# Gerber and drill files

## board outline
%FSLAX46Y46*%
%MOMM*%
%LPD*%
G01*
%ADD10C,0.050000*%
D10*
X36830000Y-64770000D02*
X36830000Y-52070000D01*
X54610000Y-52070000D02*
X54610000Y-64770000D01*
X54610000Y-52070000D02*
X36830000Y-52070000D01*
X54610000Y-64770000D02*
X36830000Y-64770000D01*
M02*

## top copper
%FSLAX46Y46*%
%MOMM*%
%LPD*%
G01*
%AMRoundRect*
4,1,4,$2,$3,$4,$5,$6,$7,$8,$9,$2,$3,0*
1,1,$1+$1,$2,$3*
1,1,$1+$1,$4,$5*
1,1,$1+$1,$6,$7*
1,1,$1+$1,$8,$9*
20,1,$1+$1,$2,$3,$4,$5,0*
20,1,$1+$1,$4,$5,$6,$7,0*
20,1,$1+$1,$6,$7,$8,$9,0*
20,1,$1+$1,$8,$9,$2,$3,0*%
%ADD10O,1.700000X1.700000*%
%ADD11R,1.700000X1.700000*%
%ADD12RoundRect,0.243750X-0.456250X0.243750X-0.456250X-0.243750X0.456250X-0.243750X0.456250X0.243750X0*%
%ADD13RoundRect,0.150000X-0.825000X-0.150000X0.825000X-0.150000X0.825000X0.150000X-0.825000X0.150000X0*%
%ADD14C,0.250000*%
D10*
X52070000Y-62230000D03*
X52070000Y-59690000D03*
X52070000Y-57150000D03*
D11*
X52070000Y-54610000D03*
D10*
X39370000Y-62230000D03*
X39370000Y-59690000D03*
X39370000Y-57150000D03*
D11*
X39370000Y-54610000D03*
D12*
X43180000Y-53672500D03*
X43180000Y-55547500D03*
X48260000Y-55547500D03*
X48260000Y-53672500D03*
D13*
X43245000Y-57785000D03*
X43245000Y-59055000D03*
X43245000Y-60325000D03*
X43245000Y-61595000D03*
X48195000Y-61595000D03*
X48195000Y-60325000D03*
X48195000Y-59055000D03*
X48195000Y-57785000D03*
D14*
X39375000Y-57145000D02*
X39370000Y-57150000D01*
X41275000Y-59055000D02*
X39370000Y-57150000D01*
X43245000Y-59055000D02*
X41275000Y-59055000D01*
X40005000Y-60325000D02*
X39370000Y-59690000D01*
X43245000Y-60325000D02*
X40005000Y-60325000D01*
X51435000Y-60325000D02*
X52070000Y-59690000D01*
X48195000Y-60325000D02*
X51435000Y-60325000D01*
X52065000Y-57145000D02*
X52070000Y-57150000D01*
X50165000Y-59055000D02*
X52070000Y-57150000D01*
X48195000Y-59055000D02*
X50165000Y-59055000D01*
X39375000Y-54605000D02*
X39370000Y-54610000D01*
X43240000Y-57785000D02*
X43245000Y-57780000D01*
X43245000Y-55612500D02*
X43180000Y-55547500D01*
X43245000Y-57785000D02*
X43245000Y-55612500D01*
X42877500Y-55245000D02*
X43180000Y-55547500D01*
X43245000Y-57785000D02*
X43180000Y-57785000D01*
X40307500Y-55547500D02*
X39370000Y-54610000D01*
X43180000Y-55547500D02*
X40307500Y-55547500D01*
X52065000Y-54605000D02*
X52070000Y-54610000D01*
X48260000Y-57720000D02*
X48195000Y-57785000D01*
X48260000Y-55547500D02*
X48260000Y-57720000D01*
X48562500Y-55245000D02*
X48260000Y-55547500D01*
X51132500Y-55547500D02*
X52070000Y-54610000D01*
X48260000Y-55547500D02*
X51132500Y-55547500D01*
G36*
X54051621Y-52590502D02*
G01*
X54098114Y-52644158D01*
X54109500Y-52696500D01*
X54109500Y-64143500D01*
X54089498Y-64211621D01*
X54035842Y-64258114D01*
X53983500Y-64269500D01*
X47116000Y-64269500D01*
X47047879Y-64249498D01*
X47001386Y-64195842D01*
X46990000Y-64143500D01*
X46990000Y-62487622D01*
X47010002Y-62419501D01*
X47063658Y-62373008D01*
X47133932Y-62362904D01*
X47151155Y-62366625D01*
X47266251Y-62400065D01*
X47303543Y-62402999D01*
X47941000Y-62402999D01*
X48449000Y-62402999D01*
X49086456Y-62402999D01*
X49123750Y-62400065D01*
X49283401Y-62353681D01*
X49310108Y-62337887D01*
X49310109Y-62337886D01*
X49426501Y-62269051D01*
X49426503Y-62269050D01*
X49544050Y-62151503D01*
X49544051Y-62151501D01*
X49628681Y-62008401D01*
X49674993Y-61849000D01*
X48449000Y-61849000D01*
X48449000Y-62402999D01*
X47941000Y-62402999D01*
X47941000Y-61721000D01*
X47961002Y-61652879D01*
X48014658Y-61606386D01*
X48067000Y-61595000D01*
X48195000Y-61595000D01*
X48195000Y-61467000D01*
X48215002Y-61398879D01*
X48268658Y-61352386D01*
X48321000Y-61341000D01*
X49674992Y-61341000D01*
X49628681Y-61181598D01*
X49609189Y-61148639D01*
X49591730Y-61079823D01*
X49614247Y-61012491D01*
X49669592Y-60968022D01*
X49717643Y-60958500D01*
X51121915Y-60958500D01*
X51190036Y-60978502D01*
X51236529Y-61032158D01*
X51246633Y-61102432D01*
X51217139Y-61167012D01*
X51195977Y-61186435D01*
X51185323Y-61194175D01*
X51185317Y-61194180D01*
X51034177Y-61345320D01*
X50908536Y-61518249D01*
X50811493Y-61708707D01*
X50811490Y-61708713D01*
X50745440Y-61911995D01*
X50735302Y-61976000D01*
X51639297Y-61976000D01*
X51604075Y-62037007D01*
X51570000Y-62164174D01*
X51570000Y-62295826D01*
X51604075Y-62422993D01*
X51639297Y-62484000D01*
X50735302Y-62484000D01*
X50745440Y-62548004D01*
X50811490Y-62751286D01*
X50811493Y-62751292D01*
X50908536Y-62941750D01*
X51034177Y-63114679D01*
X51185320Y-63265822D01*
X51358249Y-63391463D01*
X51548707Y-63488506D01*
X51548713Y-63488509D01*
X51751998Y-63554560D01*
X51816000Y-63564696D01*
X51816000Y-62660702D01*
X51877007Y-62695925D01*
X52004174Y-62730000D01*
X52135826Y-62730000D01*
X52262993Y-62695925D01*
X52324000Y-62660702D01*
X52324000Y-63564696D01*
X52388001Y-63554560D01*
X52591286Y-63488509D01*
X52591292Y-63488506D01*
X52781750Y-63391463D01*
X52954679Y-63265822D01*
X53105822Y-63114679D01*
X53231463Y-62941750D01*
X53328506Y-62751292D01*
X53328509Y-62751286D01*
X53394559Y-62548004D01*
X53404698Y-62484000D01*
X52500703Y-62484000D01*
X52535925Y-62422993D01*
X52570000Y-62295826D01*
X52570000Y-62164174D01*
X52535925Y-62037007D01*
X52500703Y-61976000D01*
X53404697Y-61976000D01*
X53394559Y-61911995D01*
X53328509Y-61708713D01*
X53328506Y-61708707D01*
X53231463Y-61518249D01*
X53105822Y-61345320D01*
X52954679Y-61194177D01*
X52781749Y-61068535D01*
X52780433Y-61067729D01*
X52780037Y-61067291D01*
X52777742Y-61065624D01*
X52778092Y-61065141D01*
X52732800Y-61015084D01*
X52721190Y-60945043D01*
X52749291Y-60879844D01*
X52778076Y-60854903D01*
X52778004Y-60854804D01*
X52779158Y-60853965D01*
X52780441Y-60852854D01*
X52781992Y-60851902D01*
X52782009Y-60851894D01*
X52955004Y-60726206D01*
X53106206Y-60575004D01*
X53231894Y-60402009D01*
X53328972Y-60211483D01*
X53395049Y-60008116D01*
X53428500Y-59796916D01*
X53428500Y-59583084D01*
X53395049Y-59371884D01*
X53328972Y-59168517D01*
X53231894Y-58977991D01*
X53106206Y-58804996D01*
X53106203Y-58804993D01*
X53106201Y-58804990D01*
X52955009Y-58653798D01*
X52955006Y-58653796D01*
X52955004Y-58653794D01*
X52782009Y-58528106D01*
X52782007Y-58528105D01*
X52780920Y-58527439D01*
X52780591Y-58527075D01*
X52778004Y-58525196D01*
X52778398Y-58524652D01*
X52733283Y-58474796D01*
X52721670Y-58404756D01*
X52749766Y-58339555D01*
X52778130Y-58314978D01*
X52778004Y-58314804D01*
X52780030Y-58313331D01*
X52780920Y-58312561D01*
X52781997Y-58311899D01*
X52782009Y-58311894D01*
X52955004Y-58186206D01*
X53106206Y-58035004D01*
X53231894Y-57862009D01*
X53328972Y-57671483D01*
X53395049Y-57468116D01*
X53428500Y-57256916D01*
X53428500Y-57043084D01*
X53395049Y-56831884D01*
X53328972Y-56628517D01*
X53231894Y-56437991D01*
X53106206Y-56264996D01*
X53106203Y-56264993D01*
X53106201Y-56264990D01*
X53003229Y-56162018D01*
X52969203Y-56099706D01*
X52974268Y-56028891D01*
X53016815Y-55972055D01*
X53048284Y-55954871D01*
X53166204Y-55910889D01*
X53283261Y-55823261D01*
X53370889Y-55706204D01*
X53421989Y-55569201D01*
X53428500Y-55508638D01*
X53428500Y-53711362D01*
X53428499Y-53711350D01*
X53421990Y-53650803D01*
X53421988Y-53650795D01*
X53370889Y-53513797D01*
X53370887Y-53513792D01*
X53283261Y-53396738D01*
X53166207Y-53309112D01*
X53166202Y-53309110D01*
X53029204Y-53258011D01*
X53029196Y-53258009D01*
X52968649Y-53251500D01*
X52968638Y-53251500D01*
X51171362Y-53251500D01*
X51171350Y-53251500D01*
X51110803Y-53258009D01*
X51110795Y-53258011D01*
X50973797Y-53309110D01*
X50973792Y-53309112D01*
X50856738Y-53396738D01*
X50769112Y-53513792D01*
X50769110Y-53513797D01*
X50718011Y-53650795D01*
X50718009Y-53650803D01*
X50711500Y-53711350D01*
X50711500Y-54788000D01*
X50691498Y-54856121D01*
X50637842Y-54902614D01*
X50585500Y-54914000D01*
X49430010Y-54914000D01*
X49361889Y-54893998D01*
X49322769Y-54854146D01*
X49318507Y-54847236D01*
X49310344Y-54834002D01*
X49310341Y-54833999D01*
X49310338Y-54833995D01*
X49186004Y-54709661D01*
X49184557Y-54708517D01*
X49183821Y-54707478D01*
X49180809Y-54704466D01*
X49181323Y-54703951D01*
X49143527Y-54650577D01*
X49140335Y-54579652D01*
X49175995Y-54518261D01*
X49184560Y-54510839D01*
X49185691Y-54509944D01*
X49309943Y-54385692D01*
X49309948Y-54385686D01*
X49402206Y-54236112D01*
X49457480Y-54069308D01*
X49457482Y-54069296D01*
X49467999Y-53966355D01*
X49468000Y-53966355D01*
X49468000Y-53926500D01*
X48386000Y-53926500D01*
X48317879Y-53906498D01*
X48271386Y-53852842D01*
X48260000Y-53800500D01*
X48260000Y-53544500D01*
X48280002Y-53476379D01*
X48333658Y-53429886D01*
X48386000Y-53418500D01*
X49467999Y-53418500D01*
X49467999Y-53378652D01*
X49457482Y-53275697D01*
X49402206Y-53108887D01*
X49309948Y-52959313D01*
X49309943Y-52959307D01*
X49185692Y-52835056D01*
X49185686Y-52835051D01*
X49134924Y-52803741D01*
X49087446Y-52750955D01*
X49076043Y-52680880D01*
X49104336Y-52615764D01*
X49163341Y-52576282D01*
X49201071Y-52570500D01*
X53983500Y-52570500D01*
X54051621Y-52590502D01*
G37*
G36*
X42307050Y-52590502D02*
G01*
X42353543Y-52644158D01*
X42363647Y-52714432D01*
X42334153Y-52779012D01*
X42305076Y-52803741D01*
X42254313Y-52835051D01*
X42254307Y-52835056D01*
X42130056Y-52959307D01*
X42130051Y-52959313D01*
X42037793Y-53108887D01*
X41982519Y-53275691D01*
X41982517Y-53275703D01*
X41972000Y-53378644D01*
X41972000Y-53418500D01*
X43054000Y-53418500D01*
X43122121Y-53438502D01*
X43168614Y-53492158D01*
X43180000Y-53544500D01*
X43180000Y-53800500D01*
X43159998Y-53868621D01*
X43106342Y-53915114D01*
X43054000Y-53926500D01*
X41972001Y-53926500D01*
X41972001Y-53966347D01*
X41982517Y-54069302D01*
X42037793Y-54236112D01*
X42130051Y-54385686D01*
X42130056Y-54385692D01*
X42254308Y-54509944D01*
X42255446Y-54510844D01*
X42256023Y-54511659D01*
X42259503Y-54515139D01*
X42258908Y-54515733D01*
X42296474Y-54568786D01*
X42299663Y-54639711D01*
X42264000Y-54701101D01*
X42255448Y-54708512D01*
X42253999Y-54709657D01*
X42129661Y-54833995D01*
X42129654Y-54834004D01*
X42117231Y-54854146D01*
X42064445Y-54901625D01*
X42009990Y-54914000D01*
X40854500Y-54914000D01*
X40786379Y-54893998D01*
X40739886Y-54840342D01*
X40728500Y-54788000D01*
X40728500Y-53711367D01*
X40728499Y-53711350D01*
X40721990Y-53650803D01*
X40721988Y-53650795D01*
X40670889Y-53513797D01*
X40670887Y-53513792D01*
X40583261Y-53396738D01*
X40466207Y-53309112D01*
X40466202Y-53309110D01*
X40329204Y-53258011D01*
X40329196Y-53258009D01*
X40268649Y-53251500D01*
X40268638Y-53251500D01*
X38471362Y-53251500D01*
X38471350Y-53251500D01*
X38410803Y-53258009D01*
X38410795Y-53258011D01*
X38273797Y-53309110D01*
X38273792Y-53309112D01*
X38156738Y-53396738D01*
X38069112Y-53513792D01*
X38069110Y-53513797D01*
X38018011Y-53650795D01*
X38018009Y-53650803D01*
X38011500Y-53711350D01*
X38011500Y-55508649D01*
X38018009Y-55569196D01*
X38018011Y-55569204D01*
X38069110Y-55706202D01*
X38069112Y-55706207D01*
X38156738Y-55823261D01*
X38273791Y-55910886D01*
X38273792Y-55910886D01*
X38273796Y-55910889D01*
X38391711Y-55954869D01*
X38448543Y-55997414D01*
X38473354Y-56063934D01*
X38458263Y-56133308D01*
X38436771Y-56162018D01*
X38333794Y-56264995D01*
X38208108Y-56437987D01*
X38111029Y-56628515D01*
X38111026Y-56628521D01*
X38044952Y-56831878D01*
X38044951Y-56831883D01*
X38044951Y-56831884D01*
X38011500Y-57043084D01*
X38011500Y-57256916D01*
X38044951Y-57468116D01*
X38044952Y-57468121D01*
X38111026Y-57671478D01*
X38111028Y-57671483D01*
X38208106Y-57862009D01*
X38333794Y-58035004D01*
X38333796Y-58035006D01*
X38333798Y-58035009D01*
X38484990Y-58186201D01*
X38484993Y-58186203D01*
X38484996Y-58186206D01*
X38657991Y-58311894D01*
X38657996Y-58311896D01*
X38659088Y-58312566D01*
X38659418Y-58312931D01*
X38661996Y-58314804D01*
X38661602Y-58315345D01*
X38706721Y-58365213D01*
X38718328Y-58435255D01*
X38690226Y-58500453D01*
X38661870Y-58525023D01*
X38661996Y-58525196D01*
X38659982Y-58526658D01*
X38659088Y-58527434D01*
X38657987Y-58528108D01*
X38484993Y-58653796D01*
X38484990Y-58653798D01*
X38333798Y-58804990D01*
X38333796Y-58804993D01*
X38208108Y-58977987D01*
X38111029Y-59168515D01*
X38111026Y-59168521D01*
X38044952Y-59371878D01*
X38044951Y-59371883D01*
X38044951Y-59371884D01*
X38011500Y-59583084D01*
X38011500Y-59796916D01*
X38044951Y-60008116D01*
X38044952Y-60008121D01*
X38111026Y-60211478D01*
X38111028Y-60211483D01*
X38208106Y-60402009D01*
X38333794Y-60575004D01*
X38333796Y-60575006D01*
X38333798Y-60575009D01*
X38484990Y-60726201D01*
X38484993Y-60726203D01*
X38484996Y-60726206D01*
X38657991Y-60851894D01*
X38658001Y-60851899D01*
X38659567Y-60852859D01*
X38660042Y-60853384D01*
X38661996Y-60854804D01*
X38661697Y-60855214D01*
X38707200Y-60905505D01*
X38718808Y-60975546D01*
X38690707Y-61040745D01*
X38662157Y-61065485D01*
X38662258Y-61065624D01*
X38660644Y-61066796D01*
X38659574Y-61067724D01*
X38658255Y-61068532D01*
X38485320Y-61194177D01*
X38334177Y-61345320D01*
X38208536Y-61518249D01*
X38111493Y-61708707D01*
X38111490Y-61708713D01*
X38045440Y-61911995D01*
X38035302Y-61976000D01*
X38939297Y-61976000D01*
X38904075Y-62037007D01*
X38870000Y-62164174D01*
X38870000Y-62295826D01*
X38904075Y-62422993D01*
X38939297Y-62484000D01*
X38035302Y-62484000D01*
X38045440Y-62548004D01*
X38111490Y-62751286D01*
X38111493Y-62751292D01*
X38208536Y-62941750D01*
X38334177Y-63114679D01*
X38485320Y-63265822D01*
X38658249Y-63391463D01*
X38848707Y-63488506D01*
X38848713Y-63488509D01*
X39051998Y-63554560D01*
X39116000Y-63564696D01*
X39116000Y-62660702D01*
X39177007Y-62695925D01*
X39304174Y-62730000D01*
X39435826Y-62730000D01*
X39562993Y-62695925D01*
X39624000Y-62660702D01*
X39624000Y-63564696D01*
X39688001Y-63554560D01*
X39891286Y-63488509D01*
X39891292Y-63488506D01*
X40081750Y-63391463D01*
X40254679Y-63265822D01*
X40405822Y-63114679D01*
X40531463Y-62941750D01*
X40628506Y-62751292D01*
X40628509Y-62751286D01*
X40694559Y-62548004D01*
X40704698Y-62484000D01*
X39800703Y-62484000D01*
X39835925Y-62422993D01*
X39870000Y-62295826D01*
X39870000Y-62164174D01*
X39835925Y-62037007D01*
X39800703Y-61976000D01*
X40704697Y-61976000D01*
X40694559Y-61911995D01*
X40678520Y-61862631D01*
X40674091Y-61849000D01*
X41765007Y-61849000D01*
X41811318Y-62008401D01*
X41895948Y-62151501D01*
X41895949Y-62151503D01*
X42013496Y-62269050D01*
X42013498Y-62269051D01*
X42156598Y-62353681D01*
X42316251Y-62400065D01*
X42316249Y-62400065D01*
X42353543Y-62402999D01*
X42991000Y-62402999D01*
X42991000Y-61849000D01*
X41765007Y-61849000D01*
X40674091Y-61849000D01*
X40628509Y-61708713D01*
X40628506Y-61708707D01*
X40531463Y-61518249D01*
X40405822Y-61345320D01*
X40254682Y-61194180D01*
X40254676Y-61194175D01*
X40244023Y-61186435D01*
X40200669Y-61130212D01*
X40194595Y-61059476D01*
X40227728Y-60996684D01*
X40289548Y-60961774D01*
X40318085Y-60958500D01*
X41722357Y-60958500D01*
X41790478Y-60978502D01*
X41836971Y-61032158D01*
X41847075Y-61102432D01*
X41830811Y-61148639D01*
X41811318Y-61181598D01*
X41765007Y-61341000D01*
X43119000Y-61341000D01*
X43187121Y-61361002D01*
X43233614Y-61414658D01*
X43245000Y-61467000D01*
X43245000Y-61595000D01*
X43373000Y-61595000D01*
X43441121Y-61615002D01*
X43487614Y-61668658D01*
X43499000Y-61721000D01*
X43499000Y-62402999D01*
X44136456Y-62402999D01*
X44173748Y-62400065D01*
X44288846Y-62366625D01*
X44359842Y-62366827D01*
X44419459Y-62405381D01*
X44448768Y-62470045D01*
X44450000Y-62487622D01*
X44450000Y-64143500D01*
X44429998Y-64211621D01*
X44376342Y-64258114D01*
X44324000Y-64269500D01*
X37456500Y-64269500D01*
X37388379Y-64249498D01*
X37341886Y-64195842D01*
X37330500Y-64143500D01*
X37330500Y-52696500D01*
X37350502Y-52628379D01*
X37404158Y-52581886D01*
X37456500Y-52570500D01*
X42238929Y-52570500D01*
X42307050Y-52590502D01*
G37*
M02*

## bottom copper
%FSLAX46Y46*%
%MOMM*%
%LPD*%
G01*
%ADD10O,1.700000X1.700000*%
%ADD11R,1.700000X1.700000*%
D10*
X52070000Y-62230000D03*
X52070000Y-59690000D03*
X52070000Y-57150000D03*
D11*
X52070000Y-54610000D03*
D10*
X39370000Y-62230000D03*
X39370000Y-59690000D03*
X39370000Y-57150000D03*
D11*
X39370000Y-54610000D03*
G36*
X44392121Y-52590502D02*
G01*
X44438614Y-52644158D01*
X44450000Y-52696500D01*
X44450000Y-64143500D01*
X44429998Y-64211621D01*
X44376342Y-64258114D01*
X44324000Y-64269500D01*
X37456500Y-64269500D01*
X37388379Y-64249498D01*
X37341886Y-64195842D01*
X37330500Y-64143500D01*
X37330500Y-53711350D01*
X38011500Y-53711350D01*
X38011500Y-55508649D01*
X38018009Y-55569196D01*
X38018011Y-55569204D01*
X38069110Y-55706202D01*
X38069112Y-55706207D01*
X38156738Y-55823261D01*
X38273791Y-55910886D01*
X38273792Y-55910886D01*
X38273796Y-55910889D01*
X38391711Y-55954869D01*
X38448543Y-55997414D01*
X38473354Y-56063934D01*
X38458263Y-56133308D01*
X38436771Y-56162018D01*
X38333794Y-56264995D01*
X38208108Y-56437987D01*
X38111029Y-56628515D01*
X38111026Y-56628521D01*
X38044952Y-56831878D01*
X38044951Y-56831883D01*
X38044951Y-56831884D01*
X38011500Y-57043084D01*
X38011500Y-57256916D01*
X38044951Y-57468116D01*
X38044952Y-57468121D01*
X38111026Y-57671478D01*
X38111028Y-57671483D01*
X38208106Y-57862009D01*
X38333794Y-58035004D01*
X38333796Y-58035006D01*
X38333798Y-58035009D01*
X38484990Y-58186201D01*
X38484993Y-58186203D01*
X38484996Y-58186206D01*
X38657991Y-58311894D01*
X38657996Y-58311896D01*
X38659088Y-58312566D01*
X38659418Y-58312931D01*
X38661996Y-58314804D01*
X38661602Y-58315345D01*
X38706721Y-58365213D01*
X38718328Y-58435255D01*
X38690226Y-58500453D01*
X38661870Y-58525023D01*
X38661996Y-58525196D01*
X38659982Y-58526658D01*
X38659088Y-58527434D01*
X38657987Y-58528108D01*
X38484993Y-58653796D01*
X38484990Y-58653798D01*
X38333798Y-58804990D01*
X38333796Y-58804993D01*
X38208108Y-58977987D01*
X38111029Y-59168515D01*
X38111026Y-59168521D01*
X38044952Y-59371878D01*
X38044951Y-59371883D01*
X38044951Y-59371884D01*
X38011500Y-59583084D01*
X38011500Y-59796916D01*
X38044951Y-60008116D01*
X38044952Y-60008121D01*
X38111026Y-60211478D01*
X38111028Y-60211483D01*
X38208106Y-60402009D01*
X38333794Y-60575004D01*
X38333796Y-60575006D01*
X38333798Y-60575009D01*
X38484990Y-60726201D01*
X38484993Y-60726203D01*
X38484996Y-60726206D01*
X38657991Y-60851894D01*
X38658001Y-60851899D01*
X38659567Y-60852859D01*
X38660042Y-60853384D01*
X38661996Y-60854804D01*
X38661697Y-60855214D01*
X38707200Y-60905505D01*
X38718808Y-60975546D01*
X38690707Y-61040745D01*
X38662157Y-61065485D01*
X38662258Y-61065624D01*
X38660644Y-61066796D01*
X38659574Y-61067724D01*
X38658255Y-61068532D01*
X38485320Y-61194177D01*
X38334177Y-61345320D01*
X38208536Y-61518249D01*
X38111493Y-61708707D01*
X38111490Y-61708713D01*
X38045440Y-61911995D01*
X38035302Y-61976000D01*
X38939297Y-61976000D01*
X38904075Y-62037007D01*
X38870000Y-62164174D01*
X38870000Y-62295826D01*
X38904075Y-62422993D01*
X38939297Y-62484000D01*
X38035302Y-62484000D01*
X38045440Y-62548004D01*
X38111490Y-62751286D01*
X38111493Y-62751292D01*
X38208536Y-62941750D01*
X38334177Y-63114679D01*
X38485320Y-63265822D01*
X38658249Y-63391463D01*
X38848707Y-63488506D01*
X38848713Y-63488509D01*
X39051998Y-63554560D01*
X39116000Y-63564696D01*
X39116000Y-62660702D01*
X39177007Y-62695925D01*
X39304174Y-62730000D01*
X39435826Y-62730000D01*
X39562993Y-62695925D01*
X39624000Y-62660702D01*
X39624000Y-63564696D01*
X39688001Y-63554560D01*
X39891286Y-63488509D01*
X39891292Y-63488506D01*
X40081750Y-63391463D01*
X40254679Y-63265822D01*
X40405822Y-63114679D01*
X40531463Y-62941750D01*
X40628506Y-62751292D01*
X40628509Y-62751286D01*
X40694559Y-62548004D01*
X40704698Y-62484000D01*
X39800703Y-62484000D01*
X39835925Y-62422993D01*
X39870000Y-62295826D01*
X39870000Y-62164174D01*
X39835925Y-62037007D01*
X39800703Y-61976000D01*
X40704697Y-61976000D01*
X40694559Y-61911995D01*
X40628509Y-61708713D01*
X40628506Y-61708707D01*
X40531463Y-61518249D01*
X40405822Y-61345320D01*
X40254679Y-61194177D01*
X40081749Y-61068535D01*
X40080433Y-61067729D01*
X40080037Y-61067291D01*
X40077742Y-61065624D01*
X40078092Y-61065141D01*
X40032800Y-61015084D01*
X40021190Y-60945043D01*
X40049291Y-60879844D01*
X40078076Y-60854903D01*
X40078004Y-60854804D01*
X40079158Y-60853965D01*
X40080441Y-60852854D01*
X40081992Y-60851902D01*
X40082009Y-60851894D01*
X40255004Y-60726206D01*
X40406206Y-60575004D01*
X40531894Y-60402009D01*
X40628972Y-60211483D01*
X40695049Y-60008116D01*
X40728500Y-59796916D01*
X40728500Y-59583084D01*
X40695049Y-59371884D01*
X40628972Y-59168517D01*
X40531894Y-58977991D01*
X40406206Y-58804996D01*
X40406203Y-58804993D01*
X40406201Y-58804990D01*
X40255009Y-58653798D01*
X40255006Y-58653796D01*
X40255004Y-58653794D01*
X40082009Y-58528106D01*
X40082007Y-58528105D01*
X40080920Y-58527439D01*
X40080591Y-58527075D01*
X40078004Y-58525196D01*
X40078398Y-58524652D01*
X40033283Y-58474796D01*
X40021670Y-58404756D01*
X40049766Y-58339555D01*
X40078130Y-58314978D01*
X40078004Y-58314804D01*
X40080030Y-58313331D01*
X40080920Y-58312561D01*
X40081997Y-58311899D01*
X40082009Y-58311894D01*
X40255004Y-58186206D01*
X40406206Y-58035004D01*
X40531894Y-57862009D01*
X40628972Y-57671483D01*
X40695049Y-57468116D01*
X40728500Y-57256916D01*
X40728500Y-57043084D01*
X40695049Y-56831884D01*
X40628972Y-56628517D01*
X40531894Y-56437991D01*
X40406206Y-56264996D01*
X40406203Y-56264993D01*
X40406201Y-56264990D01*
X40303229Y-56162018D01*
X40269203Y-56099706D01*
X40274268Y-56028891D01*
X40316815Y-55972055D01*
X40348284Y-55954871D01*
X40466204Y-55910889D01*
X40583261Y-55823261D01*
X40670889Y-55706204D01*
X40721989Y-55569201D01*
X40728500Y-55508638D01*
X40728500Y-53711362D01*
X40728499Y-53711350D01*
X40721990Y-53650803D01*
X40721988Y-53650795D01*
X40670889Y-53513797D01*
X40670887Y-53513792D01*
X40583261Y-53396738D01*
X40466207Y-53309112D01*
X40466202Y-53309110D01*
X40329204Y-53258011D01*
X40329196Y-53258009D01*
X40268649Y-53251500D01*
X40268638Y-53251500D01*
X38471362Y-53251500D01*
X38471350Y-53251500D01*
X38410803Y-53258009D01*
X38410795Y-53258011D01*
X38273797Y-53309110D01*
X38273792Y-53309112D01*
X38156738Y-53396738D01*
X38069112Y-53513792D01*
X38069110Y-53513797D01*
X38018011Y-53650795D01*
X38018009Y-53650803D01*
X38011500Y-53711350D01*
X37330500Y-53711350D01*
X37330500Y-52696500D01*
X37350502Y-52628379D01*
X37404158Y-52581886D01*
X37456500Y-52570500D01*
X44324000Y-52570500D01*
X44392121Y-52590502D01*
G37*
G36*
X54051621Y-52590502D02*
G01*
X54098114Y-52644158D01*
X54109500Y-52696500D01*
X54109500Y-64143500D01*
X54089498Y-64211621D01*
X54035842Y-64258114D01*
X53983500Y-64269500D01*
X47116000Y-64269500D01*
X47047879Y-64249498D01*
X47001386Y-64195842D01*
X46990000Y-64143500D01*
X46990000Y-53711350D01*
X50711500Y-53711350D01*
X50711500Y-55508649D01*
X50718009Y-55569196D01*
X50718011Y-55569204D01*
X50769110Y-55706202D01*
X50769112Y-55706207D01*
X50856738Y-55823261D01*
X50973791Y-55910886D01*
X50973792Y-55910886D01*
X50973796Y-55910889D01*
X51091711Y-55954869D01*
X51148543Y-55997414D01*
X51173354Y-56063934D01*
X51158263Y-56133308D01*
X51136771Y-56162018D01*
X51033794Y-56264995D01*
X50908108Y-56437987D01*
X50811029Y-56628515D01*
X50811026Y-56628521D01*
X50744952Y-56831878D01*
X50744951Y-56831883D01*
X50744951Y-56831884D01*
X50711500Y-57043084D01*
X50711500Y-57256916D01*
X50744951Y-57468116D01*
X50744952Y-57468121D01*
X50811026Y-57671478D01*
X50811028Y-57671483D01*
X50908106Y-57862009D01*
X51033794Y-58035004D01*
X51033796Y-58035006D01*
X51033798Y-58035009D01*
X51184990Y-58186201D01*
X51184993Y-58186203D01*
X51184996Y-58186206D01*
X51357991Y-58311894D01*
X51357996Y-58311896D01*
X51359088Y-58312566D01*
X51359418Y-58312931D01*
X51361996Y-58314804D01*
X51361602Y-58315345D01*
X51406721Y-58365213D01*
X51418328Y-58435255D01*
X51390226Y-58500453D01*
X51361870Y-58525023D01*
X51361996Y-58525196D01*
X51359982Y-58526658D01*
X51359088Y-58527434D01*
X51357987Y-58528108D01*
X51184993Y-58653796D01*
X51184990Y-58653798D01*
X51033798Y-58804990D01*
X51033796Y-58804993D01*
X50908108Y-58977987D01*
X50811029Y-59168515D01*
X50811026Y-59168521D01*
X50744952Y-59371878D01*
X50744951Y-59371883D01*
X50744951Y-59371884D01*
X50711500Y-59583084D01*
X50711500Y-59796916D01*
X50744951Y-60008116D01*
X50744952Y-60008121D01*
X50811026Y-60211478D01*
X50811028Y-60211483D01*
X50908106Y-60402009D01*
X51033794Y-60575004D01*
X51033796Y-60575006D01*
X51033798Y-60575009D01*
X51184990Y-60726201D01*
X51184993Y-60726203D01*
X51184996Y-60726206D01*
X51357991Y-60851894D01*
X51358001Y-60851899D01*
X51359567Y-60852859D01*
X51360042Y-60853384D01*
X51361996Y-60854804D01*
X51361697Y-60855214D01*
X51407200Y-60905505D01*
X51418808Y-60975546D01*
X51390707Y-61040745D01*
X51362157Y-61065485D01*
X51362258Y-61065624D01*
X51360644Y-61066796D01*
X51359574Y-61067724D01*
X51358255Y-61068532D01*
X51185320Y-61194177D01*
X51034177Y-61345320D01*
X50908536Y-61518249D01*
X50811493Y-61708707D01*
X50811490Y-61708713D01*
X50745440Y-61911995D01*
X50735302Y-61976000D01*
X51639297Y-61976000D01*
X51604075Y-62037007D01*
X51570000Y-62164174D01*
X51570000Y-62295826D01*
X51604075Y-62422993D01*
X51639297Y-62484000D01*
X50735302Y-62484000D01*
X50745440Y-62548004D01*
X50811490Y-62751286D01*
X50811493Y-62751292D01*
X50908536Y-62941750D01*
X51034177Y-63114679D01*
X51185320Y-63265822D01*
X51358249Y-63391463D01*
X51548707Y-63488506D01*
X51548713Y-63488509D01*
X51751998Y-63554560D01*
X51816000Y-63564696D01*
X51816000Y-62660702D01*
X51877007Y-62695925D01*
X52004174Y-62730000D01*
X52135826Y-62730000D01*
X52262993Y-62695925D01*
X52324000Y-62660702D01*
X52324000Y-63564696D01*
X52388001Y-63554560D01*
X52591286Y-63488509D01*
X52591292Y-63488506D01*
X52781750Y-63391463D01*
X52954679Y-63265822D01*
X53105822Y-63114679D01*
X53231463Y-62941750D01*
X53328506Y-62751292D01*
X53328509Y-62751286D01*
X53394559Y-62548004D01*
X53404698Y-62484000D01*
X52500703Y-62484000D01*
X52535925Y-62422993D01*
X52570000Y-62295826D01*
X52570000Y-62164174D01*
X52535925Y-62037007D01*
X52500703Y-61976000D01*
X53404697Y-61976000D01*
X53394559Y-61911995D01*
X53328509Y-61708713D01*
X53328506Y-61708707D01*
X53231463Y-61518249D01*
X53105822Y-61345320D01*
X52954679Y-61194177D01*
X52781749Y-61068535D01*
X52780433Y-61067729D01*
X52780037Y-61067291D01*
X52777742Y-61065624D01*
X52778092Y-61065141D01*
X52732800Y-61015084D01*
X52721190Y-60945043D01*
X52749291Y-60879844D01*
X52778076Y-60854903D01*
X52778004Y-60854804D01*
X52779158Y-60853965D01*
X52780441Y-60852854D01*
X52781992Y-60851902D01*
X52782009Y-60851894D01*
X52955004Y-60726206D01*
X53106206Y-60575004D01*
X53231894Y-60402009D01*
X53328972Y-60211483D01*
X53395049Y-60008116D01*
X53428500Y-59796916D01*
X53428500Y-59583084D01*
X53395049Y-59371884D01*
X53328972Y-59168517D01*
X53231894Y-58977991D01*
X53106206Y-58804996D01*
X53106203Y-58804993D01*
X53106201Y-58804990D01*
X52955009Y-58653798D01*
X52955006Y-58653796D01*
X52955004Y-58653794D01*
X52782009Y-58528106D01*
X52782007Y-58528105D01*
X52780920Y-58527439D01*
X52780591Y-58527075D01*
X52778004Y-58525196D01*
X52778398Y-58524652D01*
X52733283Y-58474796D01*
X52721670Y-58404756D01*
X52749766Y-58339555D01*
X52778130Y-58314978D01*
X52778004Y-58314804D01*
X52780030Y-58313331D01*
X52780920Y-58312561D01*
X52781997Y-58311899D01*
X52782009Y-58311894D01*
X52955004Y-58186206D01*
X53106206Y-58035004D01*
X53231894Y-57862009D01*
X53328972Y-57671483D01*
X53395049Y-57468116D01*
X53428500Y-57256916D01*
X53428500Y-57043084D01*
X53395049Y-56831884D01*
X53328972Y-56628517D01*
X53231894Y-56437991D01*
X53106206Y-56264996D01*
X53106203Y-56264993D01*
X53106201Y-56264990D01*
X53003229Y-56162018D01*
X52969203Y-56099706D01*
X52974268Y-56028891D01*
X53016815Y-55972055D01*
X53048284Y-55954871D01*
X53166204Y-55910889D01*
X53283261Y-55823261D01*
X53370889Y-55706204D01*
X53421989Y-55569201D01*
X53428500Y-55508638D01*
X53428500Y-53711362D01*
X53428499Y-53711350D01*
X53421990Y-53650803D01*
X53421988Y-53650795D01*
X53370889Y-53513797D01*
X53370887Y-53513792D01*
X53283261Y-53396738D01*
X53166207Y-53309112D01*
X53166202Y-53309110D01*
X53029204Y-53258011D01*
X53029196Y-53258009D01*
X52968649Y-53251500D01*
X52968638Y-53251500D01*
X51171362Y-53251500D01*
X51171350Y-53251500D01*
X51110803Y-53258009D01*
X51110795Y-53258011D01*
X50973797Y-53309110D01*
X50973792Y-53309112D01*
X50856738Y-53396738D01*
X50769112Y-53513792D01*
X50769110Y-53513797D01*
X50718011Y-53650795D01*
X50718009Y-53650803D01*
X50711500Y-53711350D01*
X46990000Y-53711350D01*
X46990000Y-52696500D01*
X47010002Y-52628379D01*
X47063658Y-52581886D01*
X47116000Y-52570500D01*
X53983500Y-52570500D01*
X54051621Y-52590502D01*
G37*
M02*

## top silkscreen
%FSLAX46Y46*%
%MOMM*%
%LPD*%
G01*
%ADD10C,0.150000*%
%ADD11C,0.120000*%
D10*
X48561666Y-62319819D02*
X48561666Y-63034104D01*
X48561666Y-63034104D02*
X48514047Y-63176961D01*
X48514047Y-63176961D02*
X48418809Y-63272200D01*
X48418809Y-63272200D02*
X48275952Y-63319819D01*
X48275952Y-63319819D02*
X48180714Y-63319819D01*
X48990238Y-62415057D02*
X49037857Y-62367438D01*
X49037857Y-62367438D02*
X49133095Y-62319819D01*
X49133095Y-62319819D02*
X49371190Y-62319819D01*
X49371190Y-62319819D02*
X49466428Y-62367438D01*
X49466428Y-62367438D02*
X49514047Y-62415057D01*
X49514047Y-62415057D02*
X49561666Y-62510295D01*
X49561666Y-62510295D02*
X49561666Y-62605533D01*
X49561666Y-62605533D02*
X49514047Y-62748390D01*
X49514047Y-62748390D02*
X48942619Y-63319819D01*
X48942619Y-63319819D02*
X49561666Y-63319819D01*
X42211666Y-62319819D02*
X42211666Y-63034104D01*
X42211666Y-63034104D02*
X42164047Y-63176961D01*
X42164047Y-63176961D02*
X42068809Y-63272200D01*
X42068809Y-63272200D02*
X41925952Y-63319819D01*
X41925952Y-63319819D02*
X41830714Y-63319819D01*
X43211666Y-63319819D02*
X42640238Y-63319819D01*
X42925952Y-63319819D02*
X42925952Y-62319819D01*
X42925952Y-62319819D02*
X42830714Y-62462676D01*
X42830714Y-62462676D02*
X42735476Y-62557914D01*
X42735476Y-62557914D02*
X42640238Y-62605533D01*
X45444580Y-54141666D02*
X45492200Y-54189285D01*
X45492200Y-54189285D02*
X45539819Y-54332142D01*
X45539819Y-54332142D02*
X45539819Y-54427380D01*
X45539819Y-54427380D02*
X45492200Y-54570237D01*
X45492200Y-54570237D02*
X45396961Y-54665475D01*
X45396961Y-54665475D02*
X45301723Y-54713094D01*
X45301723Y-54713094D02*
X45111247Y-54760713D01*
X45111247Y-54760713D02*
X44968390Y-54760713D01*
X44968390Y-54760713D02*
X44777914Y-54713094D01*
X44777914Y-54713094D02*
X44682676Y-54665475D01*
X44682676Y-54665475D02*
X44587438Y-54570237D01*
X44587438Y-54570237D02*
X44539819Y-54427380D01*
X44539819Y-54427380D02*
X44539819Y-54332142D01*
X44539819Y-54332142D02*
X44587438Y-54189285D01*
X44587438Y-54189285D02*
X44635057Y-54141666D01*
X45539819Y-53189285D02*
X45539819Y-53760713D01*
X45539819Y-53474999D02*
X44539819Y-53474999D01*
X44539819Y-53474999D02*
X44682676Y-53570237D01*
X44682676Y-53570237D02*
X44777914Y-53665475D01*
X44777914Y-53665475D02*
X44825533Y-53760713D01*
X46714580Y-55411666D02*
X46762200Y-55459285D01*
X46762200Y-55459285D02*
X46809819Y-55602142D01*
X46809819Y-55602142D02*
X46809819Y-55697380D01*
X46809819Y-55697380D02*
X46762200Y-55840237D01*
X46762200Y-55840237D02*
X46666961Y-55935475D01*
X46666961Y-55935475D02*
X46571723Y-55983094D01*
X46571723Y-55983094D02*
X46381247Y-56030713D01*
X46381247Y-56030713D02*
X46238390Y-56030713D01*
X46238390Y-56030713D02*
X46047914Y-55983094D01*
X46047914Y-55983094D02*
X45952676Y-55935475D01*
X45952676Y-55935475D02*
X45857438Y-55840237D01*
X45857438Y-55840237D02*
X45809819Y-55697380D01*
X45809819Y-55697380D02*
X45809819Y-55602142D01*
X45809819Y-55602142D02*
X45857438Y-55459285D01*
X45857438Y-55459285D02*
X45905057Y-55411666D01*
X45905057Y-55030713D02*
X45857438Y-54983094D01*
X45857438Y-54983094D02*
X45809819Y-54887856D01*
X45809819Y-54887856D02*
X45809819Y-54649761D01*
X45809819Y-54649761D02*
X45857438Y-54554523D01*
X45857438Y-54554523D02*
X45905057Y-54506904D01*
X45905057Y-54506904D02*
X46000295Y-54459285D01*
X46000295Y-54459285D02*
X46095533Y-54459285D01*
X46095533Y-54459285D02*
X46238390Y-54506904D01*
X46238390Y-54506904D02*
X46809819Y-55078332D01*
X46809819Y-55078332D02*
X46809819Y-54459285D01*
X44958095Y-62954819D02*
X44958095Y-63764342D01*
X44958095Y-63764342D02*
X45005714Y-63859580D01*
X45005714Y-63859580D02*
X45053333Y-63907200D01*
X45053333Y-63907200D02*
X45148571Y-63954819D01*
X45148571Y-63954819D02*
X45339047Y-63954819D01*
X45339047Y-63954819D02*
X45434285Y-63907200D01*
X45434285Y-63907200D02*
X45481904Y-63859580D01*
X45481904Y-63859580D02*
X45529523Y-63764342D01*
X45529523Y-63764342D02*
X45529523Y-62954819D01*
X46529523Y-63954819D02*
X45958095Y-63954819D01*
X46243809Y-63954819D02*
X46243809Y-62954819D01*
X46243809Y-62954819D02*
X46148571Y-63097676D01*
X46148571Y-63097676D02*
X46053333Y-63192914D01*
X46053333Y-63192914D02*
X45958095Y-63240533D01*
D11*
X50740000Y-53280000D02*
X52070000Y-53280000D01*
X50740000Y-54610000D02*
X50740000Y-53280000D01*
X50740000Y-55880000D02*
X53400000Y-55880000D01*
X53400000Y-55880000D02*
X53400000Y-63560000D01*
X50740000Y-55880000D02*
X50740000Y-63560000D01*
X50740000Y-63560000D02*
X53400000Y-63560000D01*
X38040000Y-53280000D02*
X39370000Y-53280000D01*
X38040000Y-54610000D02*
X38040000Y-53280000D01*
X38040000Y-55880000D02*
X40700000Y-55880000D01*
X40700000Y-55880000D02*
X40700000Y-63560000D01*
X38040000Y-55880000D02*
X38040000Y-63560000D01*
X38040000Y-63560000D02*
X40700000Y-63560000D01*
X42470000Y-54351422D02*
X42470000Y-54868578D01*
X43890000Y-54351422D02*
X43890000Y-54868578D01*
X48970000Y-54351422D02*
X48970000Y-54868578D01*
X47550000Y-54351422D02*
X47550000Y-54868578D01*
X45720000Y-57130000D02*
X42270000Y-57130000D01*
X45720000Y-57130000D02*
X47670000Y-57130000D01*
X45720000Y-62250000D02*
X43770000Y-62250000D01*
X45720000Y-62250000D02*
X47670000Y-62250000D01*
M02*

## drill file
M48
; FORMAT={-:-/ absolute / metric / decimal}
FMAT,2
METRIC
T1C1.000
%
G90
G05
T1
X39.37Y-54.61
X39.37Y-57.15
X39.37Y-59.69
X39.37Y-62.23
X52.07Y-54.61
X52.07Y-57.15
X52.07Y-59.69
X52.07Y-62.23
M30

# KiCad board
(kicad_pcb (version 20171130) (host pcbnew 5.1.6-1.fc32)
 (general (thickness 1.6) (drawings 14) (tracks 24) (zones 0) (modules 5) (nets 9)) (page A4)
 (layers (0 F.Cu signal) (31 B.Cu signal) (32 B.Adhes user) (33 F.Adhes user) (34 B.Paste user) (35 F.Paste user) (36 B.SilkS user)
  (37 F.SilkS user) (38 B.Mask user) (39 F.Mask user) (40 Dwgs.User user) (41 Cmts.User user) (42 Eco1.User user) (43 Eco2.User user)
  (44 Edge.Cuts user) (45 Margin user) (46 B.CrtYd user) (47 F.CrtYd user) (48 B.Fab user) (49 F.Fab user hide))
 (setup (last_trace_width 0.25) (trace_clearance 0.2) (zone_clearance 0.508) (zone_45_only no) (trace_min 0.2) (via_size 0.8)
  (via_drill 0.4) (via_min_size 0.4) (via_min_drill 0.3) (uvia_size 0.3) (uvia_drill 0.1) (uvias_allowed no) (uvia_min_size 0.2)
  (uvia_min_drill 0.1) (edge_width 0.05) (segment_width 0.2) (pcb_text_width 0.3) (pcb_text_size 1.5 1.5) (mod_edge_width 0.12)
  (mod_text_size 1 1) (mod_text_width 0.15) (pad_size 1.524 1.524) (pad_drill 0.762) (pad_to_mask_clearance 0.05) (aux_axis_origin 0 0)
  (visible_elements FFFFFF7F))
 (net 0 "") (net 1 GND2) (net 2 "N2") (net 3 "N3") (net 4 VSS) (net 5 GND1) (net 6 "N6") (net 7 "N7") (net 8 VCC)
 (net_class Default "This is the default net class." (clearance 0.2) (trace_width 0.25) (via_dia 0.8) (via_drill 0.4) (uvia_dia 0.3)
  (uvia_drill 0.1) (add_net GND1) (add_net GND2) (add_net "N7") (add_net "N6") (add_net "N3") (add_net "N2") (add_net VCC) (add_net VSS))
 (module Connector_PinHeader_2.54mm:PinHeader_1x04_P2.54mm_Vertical (layer F.Cu) (at 52.07 54.61)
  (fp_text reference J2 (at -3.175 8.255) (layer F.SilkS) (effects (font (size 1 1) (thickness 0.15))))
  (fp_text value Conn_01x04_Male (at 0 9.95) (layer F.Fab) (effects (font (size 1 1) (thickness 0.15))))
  (fp_line (start -1.33 -1.33) (end 0 -1.33) (layer F.SilkS) (width 0.12))
  (fp_line (start -1.33 0) (end -1.33 -1.33) (layer F.SilkS) (width 0.12))
  (fp_line (start -1.33 1.27) (end 1.33 1.27) (layer F.SilkS) (width 0.12))
  (fp_line (start 1.33 1.27) (end 1.33 8.95) (layer F.SilkS) (width 0.12))
  (fp_line (start -1.33 1.27) (end -1.33 8.95) (layer F.SilkS) (width 0.12))
  (fp_line (start -1.33 8.95) (end 1.33 8.95) (layer F.SilkS) (width 0.12))
  (pad 4 thru_hole oval (at 0 7.62) (size 1.7 1.7) (drill 1) (layers *.Cu *.Mask) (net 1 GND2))
  (pad 3 thru_hole oval (at 0 5.08) (size 1.7 1.7) (drill 1) (layers *.Cu *.Mask) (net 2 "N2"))
  (pad 2 thru_hole oval (at 0 2.54) (size 1.7 1.7) (drill 1) (layers *.Cu *.Mask) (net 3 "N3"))
  (pad 1 thru_hole rect (at 0 0) (size 1.7 1.7) (drill 1) (layers *.Cu *.Mask) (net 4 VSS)))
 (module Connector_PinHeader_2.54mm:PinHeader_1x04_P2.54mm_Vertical (layer F.Cu) (at 39.37 54.61)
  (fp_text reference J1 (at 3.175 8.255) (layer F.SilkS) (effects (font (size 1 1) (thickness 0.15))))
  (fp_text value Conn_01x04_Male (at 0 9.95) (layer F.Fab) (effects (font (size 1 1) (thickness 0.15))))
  (fp_line (start -1.33 -1.33) (end 0 -1.33) (layer F.SilkS) (width 0.12))
  (fp_line (start -1.33 0) (end -1.33 -1.33) (layer F.SilkS) (width 0.12))
  (fp_line (start -1.33 1.27) (end 1.33 1.27) (layer F.SilkS) (width 0.12))
  (fp_line (start 1.33 1.27) (end 1.33 8.95) (layer F.SilkS) (width 0.12))
  (fp_line (start -1.33 1.27) (end -1.33 8.95) (layer F.SilkS) (width 0.12))
  (fp_line (start -1.33 8.95) (end 1.33 8.95) (layer F.SilkS) (width 0.12))
  (pad 4 thru_hole oval (at 0 7.62) (size 1.7 1.7) (drill 1) (layers *.Cu *.Mask) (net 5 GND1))
  (pad 3 thru_hole oval (at 0 5.08) (size 1.7 1.7) (drill 1) (layers *.Cu *.Mask) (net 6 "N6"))
  (pad 2 thru_hole oval (at 0 2.54) (size 1.7 1.7) (drill 1) (layers *.Cu *.Mask) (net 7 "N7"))
  (pad 1 thru_hole rect (at 0 0) (size 1.7 1.7) (drill 1) (layers *.Cu *.Mask) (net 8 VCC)))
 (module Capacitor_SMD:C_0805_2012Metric (layer F.Cu) (at 43.18 54.61 270)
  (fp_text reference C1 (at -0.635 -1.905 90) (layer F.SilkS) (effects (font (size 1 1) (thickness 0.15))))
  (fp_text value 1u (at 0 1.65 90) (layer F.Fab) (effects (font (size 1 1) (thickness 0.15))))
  (fp_line (start -0.258578 0.71) (end 0.258578 0.71) (layer F.SilkS) (width 0.12))
  (fp_line (start -0.258578 -0.71) (end 0.258578 -0.71) (layer F.SilkS) (width 0.12))
  (pad 1 smd roundrect (at -0.9375 0 270) (size 0.975 1.4) (layers F.Cu F.Paste F.Mask) (roundrect_rratio 0.25) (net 5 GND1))
  (pad 2 smd roundrect (at 0.9375 0 270) (size 0.975 1.4) (layers F.Cu F.Paste F.Mask) (roundrect_rratio 0.25) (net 8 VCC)))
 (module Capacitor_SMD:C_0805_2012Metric (layer F.Cu) (at 48.26 54.61 270)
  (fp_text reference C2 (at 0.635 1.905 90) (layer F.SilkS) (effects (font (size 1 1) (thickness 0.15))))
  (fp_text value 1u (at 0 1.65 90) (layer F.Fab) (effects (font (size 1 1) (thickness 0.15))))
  (fp_line (start -0.258578 -0.71) (end 0.258578 -0.71) (layer F.SilkS) (width 0.12))
  (fp_line (start -0.258578 0.71) (end 0.258578 0.71) (layer F.SilkS) (width 0.12))
  (pad 2 smd roundrect (at 0.9375 0 270) (size 0.975 1.4) (layers F.Cu F.Paste F.Mask) (roundrect_rratio 0.25) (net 4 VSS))
  (pad 1 smd roundrect (at -0.9375 0 270) (size 0.975 1.4) (layers F.Cu F.Paste F.Mask) (roundrect_rratio 0.25) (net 1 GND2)))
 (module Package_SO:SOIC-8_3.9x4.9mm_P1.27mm (layer F.Cu) (at 45.72 59.69)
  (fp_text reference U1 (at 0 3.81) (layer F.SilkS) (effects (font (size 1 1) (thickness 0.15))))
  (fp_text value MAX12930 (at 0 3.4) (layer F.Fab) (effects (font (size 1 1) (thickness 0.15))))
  (fp_line (start 0 -2.56) (end -3.45 -2.56) (layer F.SilkS) (width 0.12))
  (fp_line (start 0 -2.56) (end 1.95 -2.56) (layer F.SilkS) (width 0.12))
  (fp_line (start 0 2.56) (end -1.95 2.56) (layer F.SilkS) (width 0.12))
  (fp_line (start 0 2.56) (end 1.95 2.56) (layer F.SilkS) (width 0.12))
  (pad 1 smd roundrect (at -2.475 -1.905) (size 1.95 0.6) (layers F.Cu F.Paste F.Mask) (roundrect_rratio 0.25) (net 8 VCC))
  (pad 2 smd roundrect (at -2.475 -0.635) (size 1.95 0.6) (layers F.Cu F.Paste F.Mask) (roundrect_rratio 0.25) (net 7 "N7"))
  (pad 3 smd roundrect (at -2.475 0.635) (size 1.95 0.6) (layers F.Cu F.Paste F.Mask) (roundrect_rratio 0.25) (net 6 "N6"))
  (pad 4 smd roundrect (at -2.475 1.905) (size 1.95 0.6) (layers F.Cu F.Paste F.Mask) (roundrect_rratio 0.25) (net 5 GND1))
  (pad 5 smd roundrect (at 2.475 1.905) (size 1.95 0.6) (layers F.Cu F.Paste F.Mask) (roundrect_rratio 0.25) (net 1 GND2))
  (pad 6 smd roundrect (at 2.475 0.635) (size 1.95 0.6) (layers F.Cu F.Paste F.Mask) (roundrect_rratio 0.25) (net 2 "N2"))
  (pad 7 smd roundrect (at 2.475 -0.635) (size 1.95 0.6) (layers F.Cu F.Paste F.Mask) (roundrect_rratio 0.25) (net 3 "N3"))
  (pad 8 smd roundrect (at 2.475 -1.905) (size 1.95 0.6) (layers F.Cu F.Paste F.Mask) (roundrect_rratio 0.25) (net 4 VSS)))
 (gr_line (start 36.83 64.77) (end 36.83 52.07) (layer Edge.Cuts) (width 0.05))
 (gr_line (start 54.61 52.07) (end 54.61 64.77) (layer Edge.Cuts) (width 0.05))
 (gr_line (start 54.61 52.07) (end 36.83 52.07) (layer Edge.Cuts) (width 0.05))
 (gr_line (start 54.61 64.77) (end 36.83 64.77) (layer Edge.Cuts) (width 0.05))
 (segment (start 39.375 57.145) (end 39.37 57.15) (width 0.25) (layer F.Cu) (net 7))
 (segment (start 41.275 59.055) (end 39.37 57.15) (width 0.25) (layer F.Cu) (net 7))
 (segment (start 43.245 59.055) (end 41.275 59.055) (width 0.25) (layer F.Cu) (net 7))
 (segment (start 40.005 60.325) (end 39.37 59.69) (width 0.25) (layer F.Cu) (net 6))
 (segment (start 43.245 60.325) (end 40.005 60.325) (width 0.25) (layer F.Cu) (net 6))
 (segment (start 51.435 60.325) (end 52.07 59.69) (width 0.25) (layer F.Cu) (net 2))
 (segment (start 48.195 60.325) (end 51.435 60.325) (width 0.25) (layer F.Cu) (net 2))
 (segment (start 52.065 57.145) (end 52.07 57.15) (width 0.25) (layer F.Cu) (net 3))
 (segment (start 50.165 59.055) (end 52.07 57.15) (width 0.25) (layer F.Cu) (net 3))
 (segment (start 48.195 59.055) (end 50.165 59.055) (width 0.25) (layer F.Cu) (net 3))
 (segment (start 39.375 54.605) (end 39.37 54.61) (width 0.25) (layer F.Cu) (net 8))
 (segment (start 43.24 57.785) (end 43.245 57.78) (width 0.25) (layer F.Cu) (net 8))
 (segment (start 43.245 55.6125) (end 43.18 55.5475) (width 0.25) (layer F.Cu) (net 8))
 (segment (start 43.245 57.785) (end 43.245 55.6125) (width 0.25) (layer F.Cu) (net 8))
 (segment (start 42.8775 55.245) (end 43.18 55.5475) (width 0.25) (layer F.Cu) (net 8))
 (segment (start 43.245 57.785) (end 43.18 57.785) (width 0.25) (layer F.Cu) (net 8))
 (segment (start 40.3075 55.5475) (end 39.37 54.61) (width 0.25) (layer F.Cu) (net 8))
 (segment (start 43.18 55.5475) (end 40.3075 55.5475) (width 0.25) (layer F.Cu) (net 8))
 (segment (start 52.065 54.605) (end 52.07 54.61) (width 0.25) (layer F.Cu) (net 4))
 (segment (start 48.26 57.72) (end 48.195 57.785) (width 0.25) (layer F.Cu) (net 4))
 (segment (start 48.26 55.5475) (end 48.26 57.72) (width 0.25) (layer F.Cu) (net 4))
 (segment (start 48.5625 55.245) (end 48.26 55.5475) (width 0.25) (layer F.Cu) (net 4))
 (segment (start 51.1325 55.5475) (end 52.07 54.61) (width 0.25) (layer F.Cu) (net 4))
 (segment (start 48.26 55.5475) (end 51.1325 55.5475) (width 0.25) (layer F.Cu) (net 4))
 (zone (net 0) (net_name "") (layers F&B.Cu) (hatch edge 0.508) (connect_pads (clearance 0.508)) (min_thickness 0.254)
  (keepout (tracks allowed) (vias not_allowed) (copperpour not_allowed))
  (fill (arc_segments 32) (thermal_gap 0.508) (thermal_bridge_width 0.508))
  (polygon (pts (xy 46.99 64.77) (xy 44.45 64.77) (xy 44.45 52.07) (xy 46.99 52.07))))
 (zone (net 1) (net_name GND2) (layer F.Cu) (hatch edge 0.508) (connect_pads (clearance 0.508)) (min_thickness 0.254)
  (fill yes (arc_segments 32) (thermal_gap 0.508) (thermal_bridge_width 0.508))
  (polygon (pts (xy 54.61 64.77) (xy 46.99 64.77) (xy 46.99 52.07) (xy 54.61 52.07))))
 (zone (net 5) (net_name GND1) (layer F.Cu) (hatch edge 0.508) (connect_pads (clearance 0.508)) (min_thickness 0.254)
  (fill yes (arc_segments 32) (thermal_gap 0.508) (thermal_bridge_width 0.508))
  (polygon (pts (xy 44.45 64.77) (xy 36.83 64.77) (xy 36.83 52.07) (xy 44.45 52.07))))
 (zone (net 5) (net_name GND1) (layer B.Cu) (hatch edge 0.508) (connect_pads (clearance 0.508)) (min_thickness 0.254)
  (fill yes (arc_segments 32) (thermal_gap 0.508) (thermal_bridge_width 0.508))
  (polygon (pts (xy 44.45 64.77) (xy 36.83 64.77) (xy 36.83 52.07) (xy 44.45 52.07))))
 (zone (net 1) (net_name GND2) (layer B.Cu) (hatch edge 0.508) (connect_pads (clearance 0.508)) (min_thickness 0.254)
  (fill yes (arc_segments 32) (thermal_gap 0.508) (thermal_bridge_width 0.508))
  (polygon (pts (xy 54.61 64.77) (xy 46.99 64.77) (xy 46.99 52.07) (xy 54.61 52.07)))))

